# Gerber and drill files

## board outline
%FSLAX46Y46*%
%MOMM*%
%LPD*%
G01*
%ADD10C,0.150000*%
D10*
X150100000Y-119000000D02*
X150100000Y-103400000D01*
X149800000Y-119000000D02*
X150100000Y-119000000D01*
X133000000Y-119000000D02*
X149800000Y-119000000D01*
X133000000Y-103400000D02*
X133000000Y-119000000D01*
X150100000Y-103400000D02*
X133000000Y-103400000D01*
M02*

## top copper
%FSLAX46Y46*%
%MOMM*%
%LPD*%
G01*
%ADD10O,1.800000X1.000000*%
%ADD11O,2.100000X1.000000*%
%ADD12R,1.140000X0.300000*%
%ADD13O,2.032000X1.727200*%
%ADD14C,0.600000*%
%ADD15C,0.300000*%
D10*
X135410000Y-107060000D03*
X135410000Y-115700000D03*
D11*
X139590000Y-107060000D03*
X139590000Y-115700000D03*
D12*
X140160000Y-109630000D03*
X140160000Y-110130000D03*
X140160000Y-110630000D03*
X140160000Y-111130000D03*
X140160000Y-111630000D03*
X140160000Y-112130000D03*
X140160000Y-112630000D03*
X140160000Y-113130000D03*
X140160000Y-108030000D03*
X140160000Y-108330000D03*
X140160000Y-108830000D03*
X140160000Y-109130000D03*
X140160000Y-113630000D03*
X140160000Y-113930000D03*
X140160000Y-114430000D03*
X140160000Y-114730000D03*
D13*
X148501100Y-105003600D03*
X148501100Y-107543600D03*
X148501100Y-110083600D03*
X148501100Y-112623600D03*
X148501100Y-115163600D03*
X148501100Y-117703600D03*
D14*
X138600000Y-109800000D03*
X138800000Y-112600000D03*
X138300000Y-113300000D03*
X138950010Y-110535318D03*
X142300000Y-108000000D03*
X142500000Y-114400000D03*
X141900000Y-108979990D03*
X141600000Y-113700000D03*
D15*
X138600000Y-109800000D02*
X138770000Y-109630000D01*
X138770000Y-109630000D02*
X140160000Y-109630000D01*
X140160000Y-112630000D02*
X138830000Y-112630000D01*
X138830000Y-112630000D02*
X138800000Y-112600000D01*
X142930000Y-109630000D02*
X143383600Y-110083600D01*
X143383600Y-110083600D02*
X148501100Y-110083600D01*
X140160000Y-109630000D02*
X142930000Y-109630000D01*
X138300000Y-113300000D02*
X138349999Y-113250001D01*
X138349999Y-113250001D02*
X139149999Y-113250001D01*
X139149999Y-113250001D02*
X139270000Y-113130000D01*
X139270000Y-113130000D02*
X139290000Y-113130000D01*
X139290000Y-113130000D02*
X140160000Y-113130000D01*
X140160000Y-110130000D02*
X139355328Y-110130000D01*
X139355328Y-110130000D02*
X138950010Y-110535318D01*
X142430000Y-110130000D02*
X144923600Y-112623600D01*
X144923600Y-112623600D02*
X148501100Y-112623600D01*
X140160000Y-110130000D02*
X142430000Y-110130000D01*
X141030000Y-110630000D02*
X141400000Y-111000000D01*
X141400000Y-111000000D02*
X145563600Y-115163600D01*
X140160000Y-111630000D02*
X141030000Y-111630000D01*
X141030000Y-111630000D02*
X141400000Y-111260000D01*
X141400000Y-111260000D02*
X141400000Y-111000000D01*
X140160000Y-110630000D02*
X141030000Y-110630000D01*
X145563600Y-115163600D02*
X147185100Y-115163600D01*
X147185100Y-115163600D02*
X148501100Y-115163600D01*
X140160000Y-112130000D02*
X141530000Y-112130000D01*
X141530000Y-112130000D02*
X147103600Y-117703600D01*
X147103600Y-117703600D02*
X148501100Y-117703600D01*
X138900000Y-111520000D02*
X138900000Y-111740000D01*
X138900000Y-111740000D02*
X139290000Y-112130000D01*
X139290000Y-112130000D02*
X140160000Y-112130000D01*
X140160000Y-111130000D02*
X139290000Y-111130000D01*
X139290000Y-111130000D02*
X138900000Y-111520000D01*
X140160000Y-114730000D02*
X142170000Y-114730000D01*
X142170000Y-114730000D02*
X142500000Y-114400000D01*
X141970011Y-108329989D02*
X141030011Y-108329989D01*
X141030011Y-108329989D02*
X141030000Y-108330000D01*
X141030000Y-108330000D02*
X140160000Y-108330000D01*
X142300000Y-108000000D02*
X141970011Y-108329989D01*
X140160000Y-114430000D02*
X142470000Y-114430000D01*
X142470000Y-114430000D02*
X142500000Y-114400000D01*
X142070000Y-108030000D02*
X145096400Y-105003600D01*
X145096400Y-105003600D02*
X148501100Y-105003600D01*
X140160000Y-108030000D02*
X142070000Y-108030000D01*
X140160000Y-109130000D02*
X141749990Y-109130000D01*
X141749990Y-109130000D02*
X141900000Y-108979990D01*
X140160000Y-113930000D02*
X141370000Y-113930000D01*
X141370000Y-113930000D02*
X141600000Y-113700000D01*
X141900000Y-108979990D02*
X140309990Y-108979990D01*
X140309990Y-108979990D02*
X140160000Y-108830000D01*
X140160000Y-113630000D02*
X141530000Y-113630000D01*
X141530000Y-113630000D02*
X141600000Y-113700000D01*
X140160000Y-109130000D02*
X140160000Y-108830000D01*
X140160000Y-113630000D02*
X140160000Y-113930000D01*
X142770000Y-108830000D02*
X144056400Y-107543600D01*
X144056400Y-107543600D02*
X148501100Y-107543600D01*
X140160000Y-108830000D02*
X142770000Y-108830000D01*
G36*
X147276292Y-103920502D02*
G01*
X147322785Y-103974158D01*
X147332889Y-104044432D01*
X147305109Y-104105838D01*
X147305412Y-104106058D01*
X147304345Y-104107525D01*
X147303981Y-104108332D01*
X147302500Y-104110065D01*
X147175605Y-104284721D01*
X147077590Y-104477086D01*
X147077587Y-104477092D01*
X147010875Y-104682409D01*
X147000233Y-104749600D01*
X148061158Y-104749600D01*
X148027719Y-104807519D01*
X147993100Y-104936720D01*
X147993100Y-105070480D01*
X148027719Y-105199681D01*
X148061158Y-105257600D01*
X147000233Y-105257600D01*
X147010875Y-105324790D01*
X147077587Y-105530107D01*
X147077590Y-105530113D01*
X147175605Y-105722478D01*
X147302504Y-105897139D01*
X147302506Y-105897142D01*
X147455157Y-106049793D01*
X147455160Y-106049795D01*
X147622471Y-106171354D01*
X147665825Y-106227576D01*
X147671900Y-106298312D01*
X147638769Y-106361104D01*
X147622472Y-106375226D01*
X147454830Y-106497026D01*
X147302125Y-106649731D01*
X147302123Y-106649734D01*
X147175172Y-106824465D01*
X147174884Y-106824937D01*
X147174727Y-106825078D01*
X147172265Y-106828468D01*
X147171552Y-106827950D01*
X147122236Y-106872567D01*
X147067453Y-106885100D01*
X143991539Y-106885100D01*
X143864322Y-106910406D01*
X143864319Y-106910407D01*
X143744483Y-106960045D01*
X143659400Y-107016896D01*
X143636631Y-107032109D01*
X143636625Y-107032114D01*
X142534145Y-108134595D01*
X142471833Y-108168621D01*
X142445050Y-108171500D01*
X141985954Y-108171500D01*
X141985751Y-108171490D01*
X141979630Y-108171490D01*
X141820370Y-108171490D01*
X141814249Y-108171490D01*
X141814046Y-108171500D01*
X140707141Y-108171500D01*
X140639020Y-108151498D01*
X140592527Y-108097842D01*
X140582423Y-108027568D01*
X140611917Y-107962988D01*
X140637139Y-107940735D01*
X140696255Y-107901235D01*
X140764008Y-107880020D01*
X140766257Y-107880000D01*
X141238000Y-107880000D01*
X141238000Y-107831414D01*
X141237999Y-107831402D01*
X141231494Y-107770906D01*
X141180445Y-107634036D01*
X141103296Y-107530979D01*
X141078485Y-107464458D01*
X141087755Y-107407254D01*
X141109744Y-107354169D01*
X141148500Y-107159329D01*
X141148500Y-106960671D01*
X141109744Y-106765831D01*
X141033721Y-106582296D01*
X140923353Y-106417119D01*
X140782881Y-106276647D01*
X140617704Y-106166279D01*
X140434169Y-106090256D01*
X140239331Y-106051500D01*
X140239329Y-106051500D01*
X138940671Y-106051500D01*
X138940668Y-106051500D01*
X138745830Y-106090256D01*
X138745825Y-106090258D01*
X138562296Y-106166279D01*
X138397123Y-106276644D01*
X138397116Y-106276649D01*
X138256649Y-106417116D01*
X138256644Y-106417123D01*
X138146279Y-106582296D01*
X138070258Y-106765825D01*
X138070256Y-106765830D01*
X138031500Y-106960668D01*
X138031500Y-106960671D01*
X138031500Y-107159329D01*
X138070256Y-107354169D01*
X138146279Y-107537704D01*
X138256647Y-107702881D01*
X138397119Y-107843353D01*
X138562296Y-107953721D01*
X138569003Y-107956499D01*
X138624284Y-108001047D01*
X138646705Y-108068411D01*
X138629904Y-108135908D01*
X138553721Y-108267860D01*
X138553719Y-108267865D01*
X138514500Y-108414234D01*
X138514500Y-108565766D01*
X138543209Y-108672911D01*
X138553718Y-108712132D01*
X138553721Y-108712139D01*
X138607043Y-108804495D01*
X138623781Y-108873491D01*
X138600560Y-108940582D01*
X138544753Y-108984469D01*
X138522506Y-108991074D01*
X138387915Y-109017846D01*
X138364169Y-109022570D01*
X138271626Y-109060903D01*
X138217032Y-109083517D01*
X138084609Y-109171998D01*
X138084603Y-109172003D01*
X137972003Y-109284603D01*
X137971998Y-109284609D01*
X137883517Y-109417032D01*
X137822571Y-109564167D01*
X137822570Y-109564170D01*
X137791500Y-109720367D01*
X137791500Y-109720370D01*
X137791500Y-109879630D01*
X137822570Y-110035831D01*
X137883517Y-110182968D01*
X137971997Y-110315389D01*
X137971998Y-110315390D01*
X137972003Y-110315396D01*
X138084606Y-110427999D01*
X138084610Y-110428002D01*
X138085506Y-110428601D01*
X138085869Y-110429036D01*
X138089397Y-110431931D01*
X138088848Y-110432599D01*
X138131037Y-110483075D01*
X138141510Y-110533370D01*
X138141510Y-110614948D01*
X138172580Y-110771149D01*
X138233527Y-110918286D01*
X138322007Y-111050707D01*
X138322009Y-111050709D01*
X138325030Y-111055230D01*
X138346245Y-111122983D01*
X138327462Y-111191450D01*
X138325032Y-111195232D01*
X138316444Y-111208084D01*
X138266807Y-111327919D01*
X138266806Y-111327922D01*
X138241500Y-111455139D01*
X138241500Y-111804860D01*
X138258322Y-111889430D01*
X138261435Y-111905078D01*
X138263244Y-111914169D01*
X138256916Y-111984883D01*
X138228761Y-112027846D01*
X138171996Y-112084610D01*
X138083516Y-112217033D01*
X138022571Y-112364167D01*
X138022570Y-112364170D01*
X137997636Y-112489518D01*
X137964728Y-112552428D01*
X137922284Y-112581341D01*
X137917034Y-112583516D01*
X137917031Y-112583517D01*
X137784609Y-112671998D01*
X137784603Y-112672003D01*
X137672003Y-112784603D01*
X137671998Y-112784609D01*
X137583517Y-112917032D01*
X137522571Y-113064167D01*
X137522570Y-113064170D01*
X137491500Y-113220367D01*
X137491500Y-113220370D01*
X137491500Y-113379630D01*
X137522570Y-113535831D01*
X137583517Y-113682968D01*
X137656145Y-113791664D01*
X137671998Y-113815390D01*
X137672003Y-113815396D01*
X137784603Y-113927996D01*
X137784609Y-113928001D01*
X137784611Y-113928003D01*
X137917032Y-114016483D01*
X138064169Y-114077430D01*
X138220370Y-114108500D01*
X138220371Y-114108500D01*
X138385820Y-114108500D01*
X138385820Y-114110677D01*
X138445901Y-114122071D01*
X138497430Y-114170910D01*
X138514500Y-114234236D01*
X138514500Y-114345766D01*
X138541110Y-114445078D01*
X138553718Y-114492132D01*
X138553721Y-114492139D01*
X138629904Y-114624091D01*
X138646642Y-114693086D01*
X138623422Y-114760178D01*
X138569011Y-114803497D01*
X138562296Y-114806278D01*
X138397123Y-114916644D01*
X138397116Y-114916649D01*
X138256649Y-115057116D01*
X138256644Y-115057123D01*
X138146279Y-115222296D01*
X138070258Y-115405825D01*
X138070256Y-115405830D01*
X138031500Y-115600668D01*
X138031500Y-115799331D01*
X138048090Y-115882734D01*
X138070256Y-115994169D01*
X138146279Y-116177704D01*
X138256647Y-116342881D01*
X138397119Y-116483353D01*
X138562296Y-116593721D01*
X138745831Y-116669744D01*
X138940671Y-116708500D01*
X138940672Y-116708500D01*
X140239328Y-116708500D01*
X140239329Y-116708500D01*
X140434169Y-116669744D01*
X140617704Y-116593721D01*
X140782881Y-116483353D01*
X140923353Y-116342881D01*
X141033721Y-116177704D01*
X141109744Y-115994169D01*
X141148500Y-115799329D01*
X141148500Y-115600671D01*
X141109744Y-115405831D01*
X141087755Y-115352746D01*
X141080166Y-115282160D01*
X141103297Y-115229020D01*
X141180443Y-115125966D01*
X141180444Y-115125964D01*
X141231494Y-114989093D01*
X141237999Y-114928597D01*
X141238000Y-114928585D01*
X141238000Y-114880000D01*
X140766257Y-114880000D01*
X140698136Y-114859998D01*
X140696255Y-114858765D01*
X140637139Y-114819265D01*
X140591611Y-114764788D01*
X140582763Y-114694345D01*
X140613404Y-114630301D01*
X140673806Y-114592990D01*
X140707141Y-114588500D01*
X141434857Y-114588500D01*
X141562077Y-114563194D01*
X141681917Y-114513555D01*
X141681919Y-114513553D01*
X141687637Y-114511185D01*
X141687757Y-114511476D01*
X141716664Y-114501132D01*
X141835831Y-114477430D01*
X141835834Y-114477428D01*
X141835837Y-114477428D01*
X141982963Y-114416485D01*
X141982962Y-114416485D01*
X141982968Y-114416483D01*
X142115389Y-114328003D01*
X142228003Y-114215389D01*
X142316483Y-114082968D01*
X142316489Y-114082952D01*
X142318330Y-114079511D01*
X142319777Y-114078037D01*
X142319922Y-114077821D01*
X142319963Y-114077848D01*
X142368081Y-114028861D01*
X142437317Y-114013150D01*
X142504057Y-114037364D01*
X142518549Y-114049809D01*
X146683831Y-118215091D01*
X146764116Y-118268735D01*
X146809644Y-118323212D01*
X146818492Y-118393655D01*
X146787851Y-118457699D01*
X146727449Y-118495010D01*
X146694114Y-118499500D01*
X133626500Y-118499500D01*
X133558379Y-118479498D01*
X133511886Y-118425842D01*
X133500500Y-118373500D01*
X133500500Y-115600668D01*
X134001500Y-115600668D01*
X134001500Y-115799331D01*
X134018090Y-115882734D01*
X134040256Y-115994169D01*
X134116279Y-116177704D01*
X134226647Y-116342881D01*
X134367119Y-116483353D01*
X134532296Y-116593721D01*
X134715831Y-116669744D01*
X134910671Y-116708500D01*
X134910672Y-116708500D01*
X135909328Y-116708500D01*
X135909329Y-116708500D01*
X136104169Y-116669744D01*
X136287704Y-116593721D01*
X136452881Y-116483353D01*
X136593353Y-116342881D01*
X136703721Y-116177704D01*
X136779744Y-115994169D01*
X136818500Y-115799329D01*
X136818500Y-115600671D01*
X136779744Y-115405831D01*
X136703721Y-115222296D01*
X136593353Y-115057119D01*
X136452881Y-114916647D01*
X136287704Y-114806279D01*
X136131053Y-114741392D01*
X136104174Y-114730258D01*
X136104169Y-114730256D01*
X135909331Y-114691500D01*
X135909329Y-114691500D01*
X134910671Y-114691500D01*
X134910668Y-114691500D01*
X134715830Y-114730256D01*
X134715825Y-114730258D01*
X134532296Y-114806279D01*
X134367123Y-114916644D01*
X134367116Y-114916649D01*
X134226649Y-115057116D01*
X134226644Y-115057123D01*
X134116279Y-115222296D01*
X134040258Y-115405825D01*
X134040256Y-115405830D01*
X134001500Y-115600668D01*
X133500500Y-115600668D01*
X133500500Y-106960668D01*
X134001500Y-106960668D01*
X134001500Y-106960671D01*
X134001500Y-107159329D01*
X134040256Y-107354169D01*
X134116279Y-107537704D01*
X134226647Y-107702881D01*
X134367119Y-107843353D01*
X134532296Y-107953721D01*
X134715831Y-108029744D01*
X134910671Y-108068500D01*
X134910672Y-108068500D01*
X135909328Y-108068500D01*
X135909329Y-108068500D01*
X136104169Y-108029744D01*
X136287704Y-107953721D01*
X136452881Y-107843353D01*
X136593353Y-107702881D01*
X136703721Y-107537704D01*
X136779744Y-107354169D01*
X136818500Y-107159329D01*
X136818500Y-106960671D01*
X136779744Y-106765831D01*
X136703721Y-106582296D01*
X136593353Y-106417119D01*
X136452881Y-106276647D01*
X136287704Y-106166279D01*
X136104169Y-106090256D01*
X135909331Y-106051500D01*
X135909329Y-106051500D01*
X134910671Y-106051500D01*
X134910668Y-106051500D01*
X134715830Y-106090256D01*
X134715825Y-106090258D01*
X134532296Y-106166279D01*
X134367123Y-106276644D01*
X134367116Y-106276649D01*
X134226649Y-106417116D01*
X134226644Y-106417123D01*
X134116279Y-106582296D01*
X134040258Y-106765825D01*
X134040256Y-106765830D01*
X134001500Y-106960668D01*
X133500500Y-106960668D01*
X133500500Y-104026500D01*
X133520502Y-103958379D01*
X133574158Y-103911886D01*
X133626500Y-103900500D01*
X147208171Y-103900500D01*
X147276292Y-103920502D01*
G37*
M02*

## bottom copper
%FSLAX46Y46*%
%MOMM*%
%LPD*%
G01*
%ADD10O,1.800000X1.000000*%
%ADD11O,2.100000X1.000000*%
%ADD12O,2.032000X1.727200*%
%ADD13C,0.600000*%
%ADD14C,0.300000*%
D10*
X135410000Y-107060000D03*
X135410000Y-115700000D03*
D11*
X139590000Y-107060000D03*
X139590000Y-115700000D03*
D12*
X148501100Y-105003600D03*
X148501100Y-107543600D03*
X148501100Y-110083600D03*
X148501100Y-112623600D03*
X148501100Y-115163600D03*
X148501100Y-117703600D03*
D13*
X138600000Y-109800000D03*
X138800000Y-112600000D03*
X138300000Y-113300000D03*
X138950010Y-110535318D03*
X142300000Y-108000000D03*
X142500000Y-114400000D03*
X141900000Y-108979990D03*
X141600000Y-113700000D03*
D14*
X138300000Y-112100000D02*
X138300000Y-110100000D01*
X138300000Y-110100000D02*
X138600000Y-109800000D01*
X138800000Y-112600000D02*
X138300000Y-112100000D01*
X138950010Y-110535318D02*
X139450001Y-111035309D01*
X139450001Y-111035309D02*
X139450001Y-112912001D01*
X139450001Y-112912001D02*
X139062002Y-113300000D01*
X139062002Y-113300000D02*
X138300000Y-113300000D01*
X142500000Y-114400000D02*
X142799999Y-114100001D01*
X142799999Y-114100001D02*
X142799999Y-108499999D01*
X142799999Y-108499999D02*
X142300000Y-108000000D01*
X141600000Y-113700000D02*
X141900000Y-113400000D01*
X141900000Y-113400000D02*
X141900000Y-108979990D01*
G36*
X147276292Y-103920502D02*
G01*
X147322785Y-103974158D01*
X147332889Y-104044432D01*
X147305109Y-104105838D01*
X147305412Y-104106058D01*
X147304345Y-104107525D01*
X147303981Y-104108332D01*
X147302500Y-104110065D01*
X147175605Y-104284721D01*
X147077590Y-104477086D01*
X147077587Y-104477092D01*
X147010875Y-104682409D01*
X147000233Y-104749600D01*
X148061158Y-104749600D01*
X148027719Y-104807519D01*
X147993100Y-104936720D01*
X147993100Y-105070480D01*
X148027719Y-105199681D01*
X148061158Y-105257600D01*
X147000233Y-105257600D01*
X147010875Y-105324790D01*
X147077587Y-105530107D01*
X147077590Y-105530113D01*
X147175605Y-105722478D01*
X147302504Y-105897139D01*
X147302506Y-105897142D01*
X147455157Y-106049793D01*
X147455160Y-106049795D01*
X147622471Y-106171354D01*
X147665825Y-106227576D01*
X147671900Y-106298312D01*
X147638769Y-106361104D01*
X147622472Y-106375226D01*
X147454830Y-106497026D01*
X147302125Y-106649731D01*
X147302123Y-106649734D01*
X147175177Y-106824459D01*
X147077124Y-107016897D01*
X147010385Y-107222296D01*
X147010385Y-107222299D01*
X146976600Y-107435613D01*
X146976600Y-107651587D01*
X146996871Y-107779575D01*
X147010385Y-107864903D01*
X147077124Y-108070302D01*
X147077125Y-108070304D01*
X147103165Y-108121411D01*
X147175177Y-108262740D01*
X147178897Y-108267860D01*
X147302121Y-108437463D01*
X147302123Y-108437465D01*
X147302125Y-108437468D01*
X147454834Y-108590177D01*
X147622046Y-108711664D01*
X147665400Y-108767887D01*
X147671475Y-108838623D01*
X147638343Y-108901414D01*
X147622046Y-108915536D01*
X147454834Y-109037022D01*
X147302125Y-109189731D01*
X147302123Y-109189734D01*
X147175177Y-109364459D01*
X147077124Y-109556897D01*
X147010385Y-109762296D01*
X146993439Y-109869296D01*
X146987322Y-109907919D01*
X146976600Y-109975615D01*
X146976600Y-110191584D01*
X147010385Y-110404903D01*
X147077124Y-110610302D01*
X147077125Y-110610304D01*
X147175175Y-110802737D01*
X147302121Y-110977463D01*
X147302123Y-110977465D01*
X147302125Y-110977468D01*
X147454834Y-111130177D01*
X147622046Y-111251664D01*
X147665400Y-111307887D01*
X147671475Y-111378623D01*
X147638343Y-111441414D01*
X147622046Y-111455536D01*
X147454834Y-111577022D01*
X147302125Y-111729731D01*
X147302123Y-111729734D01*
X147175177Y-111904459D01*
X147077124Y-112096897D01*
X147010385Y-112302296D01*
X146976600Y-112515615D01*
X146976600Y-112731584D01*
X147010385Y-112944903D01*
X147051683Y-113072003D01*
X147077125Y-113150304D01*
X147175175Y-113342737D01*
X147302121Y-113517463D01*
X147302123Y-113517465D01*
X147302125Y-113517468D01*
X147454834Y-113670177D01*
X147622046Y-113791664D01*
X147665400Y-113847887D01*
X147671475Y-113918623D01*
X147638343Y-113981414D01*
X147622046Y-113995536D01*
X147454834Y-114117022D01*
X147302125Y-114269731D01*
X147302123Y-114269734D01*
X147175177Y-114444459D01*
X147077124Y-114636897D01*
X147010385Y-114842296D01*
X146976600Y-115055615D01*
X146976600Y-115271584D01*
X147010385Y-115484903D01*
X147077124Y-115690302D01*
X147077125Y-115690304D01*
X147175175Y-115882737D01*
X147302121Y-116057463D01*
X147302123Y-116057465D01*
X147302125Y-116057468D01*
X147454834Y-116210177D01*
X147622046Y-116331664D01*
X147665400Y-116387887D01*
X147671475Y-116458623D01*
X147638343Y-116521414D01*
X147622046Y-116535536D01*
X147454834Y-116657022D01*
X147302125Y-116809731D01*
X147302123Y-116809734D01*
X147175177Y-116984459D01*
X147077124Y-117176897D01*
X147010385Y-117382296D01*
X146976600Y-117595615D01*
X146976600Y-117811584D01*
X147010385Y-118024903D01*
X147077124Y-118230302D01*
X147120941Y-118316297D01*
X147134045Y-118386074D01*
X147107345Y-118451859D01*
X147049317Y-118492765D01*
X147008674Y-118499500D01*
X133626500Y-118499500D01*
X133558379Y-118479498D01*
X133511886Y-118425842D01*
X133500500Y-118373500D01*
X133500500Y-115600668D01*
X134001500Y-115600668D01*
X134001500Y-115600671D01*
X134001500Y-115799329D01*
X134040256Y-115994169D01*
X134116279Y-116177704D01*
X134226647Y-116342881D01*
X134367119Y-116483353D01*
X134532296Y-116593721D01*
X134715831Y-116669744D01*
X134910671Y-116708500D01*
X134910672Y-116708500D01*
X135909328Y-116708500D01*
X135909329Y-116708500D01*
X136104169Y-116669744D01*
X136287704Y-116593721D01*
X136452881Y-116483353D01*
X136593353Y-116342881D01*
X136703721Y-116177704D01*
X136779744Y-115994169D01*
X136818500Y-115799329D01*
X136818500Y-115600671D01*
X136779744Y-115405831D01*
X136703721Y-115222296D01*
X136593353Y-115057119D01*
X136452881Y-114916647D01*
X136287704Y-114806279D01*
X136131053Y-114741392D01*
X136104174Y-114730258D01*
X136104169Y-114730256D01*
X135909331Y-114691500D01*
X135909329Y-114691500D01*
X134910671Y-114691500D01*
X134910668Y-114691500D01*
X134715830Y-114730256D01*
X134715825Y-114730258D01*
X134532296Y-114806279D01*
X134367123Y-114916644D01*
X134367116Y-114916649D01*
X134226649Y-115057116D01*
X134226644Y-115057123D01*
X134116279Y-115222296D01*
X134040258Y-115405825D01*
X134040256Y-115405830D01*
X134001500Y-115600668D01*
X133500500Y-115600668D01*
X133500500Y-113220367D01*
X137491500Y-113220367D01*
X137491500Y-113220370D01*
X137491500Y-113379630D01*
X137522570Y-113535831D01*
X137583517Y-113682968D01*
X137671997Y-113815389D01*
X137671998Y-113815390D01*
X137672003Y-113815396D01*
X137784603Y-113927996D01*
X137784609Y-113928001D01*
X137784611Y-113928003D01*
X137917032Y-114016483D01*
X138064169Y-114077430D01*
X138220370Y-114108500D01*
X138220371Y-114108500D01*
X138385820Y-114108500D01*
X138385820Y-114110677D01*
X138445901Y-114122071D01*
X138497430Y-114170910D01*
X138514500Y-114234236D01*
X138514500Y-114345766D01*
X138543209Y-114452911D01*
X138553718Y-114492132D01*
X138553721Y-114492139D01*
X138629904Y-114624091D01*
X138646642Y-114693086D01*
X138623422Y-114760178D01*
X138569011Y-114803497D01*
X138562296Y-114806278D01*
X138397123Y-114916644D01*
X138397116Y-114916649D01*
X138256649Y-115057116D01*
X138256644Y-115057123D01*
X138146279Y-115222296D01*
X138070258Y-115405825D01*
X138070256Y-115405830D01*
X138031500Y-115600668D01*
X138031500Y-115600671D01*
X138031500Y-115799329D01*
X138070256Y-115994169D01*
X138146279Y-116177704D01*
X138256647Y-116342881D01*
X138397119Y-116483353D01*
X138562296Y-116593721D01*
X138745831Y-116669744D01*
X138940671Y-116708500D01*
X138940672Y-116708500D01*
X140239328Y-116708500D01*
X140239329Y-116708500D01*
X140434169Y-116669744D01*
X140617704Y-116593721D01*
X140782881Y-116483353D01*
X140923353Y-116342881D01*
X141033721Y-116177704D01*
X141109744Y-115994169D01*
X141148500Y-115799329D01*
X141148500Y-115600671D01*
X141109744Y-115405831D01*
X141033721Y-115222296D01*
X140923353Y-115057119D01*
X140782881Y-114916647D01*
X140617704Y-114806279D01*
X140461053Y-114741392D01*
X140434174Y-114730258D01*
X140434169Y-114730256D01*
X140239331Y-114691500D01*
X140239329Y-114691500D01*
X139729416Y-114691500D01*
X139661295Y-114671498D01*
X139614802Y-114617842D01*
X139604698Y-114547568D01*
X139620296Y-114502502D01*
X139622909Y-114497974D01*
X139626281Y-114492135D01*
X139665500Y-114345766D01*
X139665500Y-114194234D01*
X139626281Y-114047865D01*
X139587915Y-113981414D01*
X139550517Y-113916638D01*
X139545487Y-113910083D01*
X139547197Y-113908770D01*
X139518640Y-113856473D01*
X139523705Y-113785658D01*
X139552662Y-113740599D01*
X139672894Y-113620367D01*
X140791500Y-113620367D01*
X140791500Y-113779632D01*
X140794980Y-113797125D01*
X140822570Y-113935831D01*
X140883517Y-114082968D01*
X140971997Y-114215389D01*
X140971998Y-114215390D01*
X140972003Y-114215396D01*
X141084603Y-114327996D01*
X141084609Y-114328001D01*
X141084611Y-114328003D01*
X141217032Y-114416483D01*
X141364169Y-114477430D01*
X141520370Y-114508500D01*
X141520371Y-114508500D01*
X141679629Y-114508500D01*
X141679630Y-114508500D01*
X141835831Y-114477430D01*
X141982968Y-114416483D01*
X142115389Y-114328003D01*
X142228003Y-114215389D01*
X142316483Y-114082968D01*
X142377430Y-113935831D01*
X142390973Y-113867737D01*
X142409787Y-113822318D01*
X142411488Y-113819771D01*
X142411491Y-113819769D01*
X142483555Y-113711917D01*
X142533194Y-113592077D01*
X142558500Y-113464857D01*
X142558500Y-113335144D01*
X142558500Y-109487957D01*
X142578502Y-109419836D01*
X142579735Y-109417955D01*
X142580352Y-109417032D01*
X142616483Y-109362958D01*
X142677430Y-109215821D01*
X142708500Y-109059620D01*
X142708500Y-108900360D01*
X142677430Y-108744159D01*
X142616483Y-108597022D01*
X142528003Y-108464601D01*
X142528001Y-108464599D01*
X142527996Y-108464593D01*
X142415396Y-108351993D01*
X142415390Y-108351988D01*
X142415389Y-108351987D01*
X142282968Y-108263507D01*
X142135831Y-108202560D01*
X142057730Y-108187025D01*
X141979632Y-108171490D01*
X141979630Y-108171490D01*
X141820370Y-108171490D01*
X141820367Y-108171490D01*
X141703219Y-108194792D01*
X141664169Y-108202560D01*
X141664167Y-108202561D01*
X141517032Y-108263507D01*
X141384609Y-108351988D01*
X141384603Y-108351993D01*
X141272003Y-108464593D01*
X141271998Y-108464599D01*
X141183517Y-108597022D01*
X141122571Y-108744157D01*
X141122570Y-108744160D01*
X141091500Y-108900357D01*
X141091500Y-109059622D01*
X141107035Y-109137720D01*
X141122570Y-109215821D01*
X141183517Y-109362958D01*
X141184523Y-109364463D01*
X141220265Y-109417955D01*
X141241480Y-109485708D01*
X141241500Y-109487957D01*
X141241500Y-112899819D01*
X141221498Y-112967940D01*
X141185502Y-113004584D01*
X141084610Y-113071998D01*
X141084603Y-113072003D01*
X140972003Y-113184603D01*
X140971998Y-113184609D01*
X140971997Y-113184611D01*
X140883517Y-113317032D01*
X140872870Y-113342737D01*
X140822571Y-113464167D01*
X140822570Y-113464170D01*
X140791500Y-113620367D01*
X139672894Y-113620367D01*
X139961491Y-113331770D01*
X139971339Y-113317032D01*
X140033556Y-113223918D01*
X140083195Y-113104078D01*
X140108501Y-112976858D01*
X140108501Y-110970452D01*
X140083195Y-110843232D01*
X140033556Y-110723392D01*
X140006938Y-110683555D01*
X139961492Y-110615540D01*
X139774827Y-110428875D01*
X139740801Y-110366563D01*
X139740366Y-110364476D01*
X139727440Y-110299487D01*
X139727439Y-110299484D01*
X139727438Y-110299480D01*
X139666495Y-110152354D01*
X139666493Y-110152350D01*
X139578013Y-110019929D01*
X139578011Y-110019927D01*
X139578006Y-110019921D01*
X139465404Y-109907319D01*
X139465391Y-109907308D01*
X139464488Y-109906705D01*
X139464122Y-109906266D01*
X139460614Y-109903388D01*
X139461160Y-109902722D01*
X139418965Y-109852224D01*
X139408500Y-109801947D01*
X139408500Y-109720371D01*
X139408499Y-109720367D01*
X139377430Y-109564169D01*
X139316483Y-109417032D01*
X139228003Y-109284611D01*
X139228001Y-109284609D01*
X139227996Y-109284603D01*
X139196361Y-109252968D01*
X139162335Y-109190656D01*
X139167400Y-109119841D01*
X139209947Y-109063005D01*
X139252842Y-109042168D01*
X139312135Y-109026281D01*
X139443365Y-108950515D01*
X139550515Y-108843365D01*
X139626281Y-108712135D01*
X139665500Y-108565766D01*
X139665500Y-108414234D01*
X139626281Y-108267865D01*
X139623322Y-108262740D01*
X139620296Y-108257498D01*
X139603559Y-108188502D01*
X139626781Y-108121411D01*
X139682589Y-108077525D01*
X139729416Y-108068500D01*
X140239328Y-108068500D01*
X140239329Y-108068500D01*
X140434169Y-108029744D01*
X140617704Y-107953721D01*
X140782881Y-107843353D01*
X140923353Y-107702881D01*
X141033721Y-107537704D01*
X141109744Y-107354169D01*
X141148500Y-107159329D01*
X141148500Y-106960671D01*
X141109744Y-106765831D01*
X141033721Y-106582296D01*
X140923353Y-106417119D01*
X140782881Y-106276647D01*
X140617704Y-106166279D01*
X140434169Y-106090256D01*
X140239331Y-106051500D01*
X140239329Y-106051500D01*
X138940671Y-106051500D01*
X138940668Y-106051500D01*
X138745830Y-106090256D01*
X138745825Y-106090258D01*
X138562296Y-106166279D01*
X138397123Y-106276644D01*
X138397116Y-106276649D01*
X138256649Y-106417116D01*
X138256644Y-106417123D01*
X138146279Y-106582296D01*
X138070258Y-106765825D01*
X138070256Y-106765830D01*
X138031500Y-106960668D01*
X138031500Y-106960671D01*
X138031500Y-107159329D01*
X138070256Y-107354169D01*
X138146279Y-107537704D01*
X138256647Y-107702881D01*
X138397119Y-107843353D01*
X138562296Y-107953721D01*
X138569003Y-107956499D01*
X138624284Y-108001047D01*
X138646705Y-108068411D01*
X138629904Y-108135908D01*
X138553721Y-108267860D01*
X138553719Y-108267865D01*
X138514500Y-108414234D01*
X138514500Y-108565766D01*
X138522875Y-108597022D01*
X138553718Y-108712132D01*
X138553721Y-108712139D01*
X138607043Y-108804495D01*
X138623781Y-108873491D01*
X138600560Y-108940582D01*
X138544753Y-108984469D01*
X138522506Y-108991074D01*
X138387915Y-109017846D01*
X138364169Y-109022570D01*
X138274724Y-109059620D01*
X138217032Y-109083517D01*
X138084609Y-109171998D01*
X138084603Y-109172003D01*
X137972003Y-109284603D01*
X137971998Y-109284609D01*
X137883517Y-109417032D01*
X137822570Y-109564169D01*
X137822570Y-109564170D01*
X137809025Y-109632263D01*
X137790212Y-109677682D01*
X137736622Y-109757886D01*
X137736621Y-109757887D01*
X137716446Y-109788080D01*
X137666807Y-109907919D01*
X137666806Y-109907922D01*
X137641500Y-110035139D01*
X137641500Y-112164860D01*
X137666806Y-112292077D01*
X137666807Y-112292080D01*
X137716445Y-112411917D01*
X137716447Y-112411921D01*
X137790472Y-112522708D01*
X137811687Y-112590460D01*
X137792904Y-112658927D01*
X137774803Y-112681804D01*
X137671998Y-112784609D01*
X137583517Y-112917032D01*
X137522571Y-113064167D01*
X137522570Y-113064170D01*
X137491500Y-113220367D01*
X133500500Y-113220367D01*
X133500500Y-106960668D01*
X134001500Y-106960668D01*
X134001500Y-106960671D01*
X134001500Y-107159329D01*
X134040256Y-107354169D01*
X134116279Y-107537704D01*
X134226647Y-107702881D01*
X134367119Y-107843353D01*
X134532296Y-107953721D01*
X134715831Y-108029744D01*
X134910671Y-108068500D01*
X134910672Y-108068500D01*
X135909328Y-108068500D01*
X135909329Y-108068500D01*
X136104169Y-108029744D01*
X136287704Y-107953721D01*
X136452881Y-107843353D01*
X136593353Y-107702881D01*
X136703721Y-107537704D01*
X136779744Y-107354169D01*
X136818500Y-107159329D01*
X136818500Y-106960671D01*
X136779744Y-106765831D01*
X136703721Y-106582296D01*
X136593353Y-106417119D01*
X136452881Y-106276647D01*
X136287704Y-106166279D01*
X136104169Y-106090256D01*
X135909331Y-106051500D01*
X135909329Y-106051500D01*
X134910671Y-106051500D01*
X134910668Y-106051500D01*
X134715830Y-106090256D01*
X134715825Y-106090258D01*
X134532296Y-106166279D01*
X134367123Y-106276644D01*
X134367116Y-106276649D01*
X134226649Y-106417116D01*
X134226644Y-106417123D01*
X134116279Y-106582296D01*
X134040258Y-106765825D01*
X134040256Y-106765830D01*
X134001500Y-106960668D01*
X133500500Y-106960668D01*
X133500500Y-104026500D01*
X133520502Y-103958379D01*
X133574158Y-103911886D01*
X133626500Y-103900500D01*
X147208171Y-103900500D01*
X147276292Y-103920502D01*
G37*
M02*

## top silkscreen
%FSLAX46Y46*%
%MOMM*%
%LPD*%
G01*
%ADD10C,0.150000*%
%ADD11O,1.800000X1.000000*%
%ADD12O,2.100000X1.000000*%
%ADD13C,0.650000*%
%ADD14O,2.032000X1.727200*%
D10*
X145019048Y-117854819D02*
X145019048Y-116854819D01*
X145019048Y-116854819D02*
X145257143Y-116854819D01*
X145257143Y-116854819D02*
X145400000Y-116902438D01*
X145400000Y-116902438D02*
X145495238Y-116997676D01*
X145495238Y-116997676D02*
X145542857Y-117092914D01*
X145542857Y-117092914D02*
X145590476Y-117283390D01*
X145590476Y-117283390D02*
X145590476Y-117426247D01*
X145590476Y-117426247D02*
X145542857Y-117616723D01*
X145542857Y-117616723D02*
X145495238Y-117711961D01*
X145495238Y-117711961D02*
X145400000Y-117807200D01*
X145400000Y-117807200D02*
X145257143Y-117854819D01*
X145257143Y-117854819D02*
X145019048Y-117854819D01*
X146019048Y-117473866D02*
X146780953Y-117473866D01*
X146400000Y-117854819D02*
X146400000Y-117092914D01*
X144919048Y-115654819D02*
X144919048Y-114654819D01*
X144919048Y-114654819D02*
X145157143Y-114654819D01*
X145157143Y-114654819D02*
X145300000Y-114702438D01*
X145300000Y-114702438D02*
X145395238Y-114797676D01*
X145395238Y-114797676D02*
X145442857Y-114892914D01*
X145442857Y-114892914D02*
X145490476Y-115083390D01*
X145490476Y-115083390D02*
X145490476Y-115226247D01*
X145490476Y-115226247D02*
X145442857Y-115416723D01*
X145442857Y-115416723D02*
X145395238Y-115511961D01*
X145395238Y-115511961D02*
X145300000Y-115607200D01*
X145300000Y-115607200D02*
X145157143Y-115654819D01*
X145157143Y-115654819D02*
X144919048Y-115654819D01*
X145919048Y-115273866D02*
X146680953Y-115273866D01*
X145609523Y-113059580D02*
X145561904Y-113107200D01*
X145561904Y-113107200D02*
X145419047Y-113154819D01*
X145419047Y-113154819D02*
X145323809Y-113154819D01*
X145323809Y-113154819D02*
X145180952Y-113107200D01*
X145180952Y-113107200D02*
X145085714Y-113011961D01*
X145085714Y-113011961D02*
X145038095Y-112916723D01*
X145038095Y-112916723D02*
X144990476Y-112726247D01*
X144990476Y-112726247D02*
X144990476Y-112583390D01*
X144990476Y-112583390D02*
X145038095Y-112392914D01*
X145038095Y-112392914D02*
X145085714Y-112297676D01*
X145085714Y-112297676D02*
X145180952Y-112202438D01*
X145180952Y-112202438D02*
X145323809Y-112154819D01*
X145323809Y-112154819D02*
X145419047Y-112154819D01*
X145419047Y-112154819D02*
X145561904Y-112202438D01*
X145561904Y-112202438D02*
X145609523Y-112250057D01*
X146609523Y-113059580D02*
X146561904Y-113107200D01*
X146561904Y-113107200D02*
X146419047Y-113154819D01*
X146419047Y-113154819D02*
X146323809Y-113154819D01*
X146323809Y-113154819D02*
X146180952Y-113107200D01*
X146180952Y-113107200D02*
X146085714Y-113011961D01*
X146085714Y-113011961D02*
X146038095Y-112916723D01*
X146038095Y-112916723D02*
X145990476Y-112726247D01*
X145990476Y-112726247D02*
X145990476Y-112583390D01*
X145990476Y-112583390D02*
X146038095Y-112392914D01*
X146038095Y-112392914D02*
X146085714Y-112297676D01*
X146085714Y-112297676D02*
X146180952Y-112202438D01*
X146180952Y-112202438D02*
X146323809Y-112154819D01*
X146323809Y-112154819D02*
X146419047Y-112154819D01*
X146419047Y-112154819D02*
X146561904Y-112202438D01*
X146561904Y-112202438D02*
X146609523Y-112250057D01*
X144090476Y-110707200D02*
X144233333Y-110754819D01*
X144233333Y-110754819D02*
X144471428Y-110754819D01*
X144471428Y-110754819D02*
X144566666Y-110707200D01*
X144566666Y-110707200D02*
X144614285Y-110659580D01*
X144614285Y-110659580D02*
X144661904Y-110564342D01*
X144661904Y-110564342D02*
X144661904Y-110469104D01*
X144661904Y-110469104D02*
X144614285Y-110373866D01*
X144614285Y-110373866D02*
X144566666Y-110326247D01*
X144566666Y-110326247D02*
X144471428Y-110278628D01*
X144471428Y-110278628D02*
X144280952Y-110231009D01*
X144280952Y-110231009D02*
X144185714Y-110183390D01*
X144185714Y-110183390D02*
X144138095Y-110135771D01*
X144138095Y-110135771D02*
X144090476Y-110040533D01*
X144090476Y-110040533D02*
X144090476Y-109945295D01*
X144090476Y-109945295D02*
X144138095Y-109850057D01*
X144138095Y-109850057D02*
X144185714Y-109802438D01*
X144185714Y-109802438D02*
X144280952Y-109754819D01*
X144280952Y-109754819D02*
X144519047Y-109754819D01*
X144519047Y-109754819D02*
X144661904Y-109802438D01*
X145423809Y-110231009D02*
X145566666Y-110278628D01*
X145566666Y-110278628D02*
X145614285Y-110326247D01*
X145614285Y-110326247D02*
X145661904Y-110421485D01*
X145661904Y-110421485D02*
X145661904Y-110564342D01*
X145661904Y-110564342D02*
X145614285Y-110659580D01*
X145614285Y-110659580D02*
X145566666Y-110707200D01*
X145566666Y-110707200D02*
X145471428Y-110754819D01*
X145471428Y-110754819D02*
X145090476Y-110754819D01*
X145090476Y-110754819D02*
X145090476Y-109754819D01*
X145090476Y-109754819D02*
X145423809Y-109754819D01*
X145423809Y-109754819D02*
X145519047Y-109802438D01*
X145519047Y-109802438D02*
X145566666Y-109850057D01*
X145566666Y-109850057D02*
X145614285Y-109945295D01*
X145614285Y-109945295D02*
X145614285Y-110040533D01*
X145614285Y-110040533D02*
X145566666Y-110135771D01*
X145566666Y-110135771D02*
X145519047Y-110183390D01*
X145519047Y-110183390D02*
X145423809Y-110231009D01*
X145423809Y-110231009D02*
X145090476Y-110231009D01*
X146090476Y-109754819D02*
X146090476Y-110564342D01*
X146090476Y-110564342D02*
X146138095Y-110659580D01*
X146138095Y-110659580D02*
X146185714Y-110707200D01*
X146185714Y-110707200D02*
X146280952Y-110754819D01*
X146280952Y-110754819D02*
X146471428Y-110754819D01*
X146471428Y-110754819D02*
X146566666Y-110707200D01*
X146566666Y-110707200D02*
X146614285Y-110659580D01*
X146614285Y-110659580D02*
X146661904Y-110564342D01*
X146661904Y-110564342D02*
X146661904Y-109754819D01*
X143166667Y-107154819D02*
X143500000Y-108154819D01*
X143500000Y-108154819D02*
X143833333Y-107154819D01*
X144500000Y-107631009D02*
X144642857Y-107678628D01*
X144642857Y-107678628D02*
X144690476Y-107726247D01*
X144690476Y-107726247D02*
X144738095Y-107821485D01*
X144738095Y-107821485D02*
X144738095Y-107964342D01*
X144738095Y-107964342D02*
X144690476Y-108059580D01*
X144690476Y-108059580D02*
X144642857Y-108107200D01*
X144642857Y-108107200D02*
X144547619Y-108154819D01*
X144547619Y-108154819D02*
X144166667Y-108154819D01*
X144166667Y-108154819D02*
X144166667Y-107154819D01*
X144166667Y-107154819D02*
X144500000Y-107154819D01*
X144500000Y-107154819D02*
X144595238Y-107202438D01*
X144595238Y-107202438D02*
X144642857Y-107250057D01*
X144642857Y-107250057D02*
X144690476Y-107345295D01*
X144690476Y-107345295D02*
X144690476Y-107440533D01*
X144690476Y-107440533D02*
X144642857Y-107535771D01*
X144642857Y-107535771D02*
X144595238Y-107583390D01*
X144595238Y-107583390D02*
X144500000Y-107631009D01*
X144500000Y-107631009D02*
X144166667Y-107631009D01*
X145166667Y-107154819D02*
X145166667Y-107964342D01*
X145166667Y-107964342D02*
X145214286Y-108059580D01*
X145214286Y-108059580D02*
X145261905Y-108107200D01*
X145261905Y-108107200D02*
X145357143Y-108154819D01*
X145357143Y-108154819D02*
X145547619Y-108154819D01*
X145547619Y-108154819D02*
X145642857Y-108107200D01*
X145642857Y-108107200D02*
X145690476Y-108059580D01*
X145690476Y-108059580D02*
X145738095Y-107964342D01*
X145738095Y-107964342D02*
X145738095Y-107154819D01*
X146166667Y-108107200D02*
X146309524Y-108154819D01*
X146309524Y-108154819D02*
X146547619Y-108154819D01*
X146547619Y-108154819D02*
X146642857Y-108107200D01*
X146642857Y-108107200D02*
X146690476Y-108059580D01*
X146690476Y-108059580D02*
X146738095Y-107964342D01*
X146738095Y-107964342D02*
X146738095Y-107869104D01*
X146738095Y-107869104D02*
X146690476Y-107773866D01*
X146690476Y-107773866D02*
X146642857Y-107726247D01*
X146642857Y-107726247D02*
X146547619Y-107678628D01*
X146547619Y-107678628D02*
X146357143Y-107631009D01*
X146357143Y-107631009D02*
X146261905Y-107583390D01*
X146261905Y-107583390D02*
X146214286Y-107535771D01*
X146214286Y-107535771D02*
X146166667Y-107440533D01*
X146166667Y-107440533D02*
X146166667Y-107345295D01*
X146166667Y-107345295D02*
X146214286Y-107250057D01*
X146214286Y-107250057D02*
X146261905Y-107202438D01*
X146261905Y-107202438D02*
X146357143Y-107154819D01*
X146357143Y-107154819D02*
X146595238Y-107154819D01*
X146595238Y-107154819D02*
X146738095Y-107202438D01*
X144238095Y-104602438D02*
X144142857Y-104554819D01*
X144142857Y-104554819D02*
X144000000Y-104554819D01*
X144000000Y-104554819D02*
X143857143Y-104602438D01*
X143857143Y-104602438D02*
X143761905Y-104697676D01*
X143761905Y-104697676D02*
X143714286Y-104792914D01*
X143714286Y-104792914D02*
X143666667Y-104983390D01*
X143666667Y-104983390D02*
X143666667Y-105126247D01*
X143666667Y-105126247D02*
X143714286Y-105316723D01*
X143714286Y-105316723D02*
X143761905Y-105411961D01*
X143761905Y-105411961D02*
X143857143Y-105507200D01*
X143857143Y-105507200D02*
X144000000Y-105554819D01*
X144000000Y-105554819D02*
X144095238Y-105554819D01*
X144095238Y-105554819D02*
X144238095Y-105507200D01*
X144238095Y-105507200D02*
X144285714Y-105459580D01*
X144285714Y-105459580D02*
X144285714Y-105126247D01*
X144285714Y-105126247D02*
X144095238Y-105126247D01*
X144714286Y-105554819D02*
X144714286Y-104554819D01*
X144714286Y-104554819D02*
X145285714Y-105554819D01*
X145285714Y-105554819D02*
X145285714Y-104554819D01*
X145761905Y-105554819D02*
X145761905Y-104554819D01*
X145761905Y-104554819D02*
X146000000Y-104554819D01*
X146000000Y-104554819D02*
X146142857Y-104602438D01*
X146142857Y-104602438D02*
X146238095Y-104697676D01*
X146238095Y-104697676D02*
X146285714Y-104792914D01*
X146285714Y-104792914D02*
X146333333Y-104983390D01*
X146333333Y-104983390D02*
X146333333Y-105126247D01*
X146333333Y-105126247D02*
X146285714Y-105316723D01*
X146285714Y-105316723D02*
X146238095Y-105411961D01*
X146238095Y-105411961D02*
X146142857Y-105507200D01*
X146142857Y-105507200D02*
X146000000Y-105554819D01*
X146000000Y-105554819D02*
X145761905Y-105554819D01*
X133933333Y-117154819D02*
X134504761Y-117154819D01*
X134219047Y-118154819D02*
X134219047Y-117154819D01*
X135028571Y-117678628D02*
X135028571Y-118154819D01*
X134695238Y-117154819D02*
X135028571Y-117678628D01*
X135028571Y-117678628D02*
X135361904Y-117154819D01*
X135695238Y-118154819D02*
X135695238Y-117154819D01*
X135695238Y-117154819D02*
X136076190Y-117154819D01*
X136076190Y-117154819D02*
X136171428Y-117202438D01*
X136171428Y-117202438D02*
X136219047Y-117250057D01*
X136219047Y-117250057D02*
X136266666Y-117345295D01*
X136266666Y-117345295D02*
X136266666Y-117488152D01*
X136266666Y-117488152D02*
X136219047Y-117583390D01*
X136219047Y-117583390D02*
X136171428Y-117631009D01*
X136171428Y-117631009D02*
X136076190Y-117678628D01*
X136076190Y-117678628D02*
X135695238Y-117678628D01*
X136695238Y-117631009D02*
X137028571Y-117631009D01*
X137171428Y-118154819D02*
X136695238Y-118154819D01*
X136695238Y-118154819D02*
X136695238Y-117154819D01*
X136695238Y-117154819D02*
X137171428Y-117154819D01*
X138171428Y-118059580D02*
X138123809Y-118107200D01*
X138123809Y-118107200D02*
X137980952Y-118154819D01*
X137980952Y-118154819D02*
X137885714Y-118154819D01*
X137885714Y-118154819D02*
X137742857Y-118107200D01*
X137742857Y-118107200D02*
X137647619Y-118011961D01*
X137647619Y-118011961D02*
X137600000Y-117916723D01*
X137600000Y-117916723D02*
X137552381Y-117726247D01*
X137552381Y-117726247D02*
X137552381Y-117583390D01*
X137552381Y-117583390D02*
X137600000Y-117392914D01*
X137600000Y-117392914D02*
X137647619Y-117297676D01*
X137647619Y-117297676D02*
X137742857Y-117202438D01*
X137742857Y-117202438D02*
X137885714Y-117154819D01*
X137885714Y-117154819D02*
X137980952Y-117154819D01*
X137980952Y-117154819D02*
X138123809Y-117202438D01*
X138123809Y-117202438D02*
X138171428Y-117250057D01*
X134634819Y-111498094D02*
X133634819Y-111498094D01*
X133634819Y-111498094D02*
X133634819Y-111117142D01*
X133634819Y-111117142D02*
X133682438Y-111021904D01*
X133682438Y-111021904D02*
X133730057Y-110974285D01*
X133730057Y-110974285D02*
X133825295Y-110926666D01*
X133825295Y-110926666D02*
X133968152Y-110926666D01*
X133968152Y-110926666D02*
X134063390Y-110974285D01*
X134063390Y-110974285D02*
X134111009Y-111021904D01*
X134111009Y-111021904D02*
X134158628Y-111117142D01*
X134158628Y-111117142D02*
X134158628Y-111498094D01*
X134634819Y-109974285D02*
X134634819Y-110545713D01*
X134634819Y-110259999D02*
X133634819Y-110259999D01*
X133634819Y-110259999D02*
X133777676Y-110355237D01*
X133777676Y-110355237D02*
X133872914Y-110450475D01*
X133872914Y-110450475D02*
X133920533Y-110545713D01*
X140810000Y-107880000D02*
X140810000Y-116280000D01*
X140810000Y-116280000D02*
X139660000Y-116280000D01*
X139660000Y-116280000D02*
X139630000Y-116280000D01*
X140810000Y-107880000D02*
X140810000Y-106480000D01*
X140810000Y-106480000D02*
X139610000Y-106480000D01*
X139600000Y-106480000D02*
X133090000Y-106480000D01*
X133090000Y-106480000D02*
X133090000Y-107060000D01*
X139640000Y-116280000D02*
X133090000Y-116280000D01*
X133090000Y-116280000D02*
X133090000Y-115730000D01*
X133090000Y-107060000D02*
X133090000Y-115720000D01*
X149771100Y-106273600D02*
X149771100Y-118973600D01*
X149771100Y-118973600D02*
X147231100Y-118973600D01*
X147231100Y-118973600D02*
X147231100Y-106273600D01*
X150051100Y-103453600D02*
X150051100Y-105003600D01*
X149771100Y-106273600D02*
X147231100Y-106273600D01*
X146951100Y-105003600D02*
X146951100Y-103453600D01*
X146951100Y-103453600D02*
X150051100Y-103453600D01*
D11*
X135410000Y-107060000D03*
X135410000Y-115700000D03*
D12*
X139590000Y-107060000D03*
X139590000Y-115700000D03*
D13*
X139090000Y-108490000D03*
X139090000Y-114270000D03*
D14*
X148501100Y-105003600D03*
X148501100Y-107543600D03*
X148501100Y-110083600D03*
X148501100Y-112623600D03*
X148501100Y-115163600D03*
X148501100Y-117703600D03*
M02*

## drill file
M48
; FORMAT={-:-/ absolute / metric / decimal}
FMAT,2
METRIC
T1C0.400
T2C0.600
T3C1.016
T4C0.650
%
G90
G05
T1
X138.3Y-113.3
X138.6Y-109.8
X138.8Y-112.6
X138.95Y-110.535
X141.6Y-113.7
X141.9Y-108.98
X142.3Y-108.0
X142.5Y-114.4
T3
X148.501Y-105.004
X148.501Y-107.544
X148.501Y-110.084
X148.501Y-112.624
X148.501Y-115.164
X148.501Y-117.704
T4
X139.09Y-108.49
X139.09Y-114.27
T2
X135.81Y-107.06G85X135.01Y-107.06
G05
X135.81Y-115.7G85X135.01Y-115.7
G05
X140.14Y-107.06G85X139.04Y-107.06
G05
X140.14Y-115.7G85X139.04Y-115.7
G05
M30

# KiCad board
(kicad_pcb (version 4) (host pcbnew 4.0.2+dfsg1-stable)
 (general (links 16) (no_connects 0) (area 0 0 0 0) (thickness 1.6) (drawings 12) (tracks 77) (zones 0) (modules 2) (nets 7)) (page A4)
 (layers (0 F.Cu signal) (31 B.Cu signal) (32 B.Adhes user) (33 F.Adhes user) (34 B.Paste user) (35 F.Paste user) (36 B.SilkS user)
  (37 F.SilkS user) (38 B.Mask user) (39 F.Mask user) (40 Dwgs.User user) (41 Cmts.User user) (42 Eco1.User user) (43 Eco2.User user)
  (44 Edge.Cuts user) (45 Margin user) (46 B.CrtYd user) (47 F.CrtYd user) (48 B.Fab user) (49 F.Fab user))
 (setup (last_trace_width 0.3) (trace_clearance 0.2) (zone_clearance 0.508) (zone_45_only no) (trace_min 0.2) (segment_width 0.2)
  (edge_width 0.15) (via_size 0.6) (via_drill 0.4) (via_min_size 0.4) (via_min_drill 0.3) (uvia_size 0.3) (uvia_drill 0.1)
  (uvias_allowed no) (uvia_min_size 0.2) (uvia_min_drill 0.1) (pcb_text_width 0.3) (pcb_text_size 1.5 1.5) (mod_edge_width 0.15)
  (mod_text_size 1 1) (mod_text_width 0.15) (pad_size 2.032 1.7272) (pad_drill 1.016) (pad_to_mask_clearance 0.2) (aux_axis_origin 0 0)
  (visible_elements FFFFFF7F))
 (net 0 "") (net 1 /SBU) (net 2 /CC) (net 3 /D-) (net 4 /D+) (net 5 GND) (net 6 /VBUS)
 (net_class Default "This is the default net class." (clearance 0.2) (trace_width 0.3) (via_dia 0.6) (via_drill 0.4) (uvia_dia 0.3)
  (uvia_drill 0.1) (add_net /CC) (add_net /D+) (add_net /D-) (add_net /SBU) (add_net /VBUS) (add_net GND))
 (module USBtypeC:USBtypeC (layer F.Cu) (at 136.8 111.7 270)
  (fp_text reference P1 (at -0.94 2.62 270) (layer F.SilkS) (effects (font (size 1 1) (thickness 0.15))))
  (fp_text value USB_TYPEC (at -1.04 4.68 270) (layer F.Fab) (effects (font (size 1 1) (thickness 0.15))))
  (fp_line (start -3.82 -4.01) (end 4.58 -4.01) (layer F.SilkS) (width 0.15))
  (fp_line (start 4.58 -4.01) (end 4.58 -2.86) (layer F.SilkS) (width 0.15))
  (fp_line (start 4.58 -2.86) (end 4.58 -2.83) (layer F.SilkS) (width 0.15))
  (fp_line (start -3.82 -4.01) (end -5.22 -4.01) (layer F.SilkS) (width 0.15))
  (fp_line (start -5.22 -4.01) (end -5.22 -2.81) (layer F.SilkS) (width 0.15))
  (fp_line (start -5.22 -2.8) (end -5.22 3.71) (layer F.SilkS) (width 0.15))
  (fp_line (start -5.22 3.71) (end -4.64 3.71) (layer F.SilkS) (width 0.15))
  (fp_line (start 4.58 -2.84) (end 4.58 3.71) (layer F.SilkS) (width 0.15))
  (fp_line (start 4.58 3.71) (end 4.03 3.71) (layer F.SilkS) (width 0.15))
  (fp_line (start -4.64 3.71) (end 4.02 3.71) (layer F.SilkS) (width 0.15))
  (pad 1 thru_hole oval (at -4.64 1.39 270) (size 1 1.8) (drill oval 0.6 1.4) (layers *.Cu *.Mask F.SilkS))
  (pad 2 thru_hole oval (at 4 1.39 270) (size 1 1.8) (drill oval 0.6 1.4) (layers *.Cu *.Mask F.SilkS))
  (pad 3 thru_hole oval (at -4.64 -2.79 270) (size 1 2.1) (drill oval 0.6 1.7) (layers *.Cu *.Mask F.SilkS))
  (pad 4 thru_hole oval (at 4 -2.79 270) (size 1 2.1) (drill oval 0.6 1.7) (layers *.Cu *.Mask F.SilkS))
  (pad "" np_thru_hole circle (at -3.21 -2.29 270) (size 0.65 0.65) (drill 0.65) (layers *.Cu *.Mask F.SilkS))
  (pad "" np_thru_hole circle (at 2.57 -2.29 270) (size 0.65 0.65) (drill 0.65) (layers *.Cu *.Mask F.SilkS))
  (pad B8 smd rect (at -2.07 -3.36 270) (size 0.3 1.14) (layers F.Cu F.Paste F.Mask) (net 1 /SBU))
  (pad A5 smd rect (at -1.57 -3.36 270) (size 0.3 1.14) (layers F.Cu F.Paste F.Mask) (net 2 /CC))
  (pad B7 smd rect (at -1.07 -3.36 270) (size 0.3 1.14) (layers F.Cu F.Paste F.Mask) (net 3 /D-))
  (pad A6 smd rect (at -0.57 -3.36 270) (size 0.3 1.14) (layers F.Cu F.Paste F.Mask) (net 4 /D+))
  (pad A7 smd rect (at -0.07 -3.36 270) (size 0.3 1.14) (layers F.Cu F.Paste F.Mask) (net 3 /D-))
  (pad B6 smd rect (at 0.43 -3.36 270) (size 0.3 1.14) (layers F.Cu F.Paste F.Mask) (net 4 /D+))
  (pad A8 smd rect (at 0.93 -3.36 270) (size 0.3 1.14) (layers F.Cu F.Paste F.Mask) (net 1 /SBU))
  (pad B5 smd rect (at 1.43 -3.36 270) (size 0.3 1.14) (layers F.Cu F.Paste F.Mask) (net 2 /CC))
  (pad A1 smd rect (at -3.67 -3.36 270) (size 0.3 1.14) (layers F.Cu F.Paste F.Mask) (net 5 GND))
  (pad B12 smd rect (at -3.37 -3.36 270) (size 0.3 1.14) (layers F.Cu F.Paste F.Mask) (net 5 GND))
  (pad A4 smd rect (at -2.87 -3.36 270) (size 0.3 1.14) (layers F.Cu F.Paste F.Mask) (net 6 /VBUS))
  (pad B9 smd rect (at -2.57 -3.36 270) (size 0.3 1.14) (layers F.Cu F.Paste F.Mask) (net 6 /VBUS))
  (pad B4 smd rect (at 1.93 -3.36 270) (size 0.3 1.14) (layers F.Cu F.Paste F.Mask) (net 6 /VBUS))
  (pad A9 smd rect (at 2.23 -3.36 270) (size 0.3 1.14) (layers F.Cu F.Paste F.Mask) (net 6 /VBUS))
  (pad B1 smd rect (at 2.73 -3.36 270) (size 0.3 1.14) (layers F.Cu F.Paste F.Mask) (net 5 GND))
  (pad A12 smd rect (at 3.03 -3.36 270) (size 0.3 1.14) (layers F.Cu F.Paste F.Mask) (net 5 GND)))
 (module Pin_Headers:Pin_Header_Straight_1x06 (layer F.Cu) (at 148.5011 105.0036)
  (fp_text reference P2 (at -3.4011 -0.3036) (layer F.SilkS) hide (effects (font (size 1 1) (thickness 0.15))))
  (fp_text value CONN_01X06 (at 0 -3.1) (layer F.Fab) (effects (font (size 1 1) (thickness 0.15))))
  (fp_line (start 1.27 1.27) (end 1.27 13.97) (layer F.SilkS) (width 0.15))
  (fp_line (start 1.27 13.97) (end -1.27 13.97) (layer F.SilkS) (width 0.15))
  (fp_line (start -1.27 13.97) (end -1.27 1.27) (layer F.SilkS) (width 0.15))
  (fp_line (start 1.55 -1.55) (end 1.55 0) (layer F.SilkS) (width 0.15))
  (fp_line (start 1.27 1.27) (end -1.27 1.27) (layer F.SilkS) (width 0.15))
  (fp_line (start -1.55 0) (end -1.55 -1.55) (layer F.SilkS) (width 0.15))
  (fp_line (start -1.55 -1.55) (end 1.55 -1.55) (layer F.SilkS) (width 0.15))
  (pad 1 thru_hole oval (at 0 0) (size 2.032 1.7272) (drill 1.016) (layers *.Cu *.Mask F.SilkS) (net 5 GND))
  (pad 2 thru_hole oval (at 0 2.54) (size 2.032 1.7272) (drill 1.016) (layers *.Cu *.Mask F.SilkS) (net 6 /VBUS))
  (pad 3 thru_hole oval (at 0 5.08) (size 2.032 1.7272) (drill 1.016) (layers *.Cu *.Mask F.SilkS) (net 1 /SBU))
  (pad 4 thru_hole oval (at 0 7.62) (size 2.032 1.7272) (drill 1.016) (layers *.Cu *.Mask F.SilkS) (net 2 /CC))
  (pad 5 thru_hole oval (at 0 10.16) (size 2.032 1.7272) (drill 1.016) (layers *.Cu *.Mask F.SilkS) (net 3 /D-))
  (pad 6 thru_hole oval (at 0 12.7) (size 2.032 1.7272) (drill 1.016) (layers *.Cu *.Mask F.SilkS) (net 4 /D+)))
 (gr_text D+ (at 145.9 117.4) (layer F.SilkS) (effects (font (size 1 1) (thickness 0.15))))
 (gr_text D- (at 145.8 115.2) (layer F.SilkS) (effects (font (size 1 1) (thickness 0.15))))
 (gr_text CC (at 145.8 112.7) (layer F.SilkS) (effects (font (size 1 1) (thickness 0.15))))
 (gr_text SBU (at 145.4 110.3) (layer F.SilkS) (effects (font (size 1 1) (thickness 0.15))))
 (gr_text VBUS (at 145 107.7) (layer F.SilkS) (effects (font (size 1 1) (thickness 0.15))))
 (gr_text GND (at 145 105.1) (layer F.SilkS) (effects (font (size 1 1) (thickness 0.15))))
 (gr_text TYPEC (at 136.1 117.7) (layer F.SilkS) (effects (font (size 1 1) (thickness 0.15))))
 (gr_line (start 150.1 119) (end 150.1 103.4) (angle 90) (layer Edge.Cuts) (width 0.15))
 (gr_line (start 149.8 119) (end 150.1 119) (angle 90) (layer Edge.Cuts) (width 0.15))
 (gr_line (start 133 119) (end 149.8 119) (angle 90) (layer Edge.Cuts) (width 0.15))
 (gr_line (start 133 103.4) (end 133 119) (angle 90) (layer Edge.Cuts) (width 0.15))
 (gr_line (start 150.1 103.4) (end 133 103.4) (angle 90) (layer Edge.Cuts) (width 0.15))
 (segment (start 138.6 109.8) (end 138.77 109.63) (width 0.3) (layer F.Cu) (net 1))
 (segment (start 138.77 109.63) (end 140.16 109.63) (width 0.3) (layer F.Cu) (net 1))
 (segment (start 138.3 112.1) (end 138.3 110.1) (width 0.3) (layer B.Cu) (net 1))
 (segment (start 138.3 110.1) (end 138.6 109.8) (width 0.3) (layer B.Cu) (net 1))
 (via (at 138.6 109.8) (size 0.6) (drill 0.4) (layers F.Cu B.Cu) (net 1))
 (segment (start 138.8 112.6) (end 138.3 112.1) (width 0.3) (layer B.Cu) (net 1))
 (segment (start 140.16 112.63) (end 138.83 112.63) (width 0.3) (layer F.Cu) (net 1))
 (segment (start 138.83 112.63) (end 138.8 112.6) (width 0.3) (layer F.Cu) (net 1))
 (via (at 138.8 112.6) (size 0.6) (drill 0.4) (layers F.Cu B.Cu) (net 1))
 (segment (start 142.93 109.63) (end 143.3836 110.0836) (width 0.3) (layer F.Cu) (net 1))
 (segment (start 143.3836 110.0836) (end 148.5011 110.0836) (width 0.3) (layer F.Cu) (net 1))
 (segment (start 140.16 109.63) (end 142.93 109.63) (width 0.3) (layer F.Cu) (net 1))
 (segment (start 138.3 113.3) (end 138.349999 113.250001) (width 0.3) (layer F.Cu) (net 2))
 (segment (start 138.349999 113.250001) (end 139.149999 113.250001) (width 0.3) (layer F.Cu) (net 2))
 (segment (start 139.149999 113.250001) (end 139.27 113.13) (width 0.3) (layer F.Cu) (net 2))
 (segment (start 139.27 113.13) (end 139.29 113.13) (width 0.3) (layer F.Cu) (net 2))
 (segment (start 139.29 113.13) (end 140.16 113.13) (width 0.3) (layer F.Cu) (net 2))
 (segment (start 138.95001 110.535318) (end 139.450001 111.035309) (width 0.3) (layer B.Cu) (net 2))
 (segment (start 139.450001 111.035309) (end 139.450001 112.912001) (width 0.3) (layer B.Cu) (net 2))
 (segment (start 139.450001 112.912001) (end 139.062002 113.3) (width 0.3) (layer B.Cu) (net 2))
 (segment (start 139.062002 113.3) (end 138.3 113.3) (width 0.3) (layer B.Cu) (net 2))
 (via (at 138.3 113.3) (size 0.6) (drill 0.4) (layers F.Cu B.Cu) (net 2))
 (segment (start 140.16 110.13) (end 139.355328 110.13) (width 0.3) (layer F.Cu) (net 2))
 (segment (start 139.355328 110.13) (end 138.95001 110.535318) (width 0.3) (layer F.Cu) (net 2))
 (via (at 138.95001 110.535318) (size 0.6) (drill 0.4) (layers F.Cu B.Cu) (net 2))
 (segment (start 142.43 110.13) (end 144.9236 112.6236) (width 0.3) (layer F.Cu) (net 2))
 (segment (start 144.9236 112.6236) (end 148.5011 112.6236) (width 0.3) (layer F.Cu) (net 2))
 (segment (start 140.16 110.13) (end 142.43 110.13) (width 0.3) (layer F.Cu) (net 2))
 (segment (start 141.03 110.63) (end 141.4 111) (width 0.3) (layer F.Cu) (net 3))
 (segment (start 141.4 111) (end 145.5636 115.1636) (width 0.3) (layer F.Cu) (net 3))
 (segment (start 140.16 111.63) (end 141.03 111.63) (width 0.3) (layer F.Cu) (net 3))
 (segment (start 141.03 111.63) (end 141.4 111.26) (width 0.3) (layer F.Cu) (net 3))
 (segment (start 141.4 111.26) (end 141.4 111) (width 0.3) (layer F.Cu) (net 3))
 (segment (start 140.16 110.63) (end 141.03 110.63) (width 0.3) (layer F.Cu) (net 3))
 (segment (start 145.5636 115.1636) (end 147.1851 115.1636) (width 0.3) (layer F.Cu) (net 3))
 (segment (start 147.1851 115.1636) (end 148.5011 115.1636) (width 0.3) (layer F.Cu) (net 3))
 (segment (start 140.16 112.13) (end 141.53 112.13) (width 0.3) (layer F.Cu) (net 4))
 (segment (start 141.53 112.13) (end 147.1036 117.7036) (width 0.3) (layer F.Cu) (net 4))
 (segment (start 147.1036 117.7036) (end 148.5011 117.7036) (width 0.3) (layer F.Cu) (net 4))
 (segment (start 138.9 111.52) (end 138.9 111.74) (width 0.3) (layer F.Cu) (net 4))
 (segment (start 138.9 111.74) (end 139.29 112.13) (width 0.3) (layer F.Cu) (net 4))
 (segment (start 139.29 112.13) (end 140.16 112.13) (width 0.3) (layer F.Cu) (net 4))
 (segment (start 140.16 111.13) (end 139.29 111.13) (width 0.3) (layer F.Cu) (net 4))
 (segment (start 139.29 111.13) (end 138.9 111.52) (width 0.3) (layer F.Cu) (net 4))
 (segment (start 140.16 114.73) (end 142.17 114.73) (width 0.3) (layer F.Cu) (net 5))
 (segment (start 142.17 114.73) (end 142.5 114.4) (width 0.3) (layer F.Cu) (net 5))
 (segment (start 141.970011 108.329989) (end 141.030011 108.329989) (width 0.3) (layer F.Cu) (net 5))
 (segment (start 141.030011 108.329989) (end 141.03 108.33) (width 0.3) (layer F.Cu) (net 5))
 (segment (start 141.03 108.33) (end 140.16 108.33) (width 0.3) (layer F.Cu) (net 5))
 (segment (start 142.3 108) (end 141.970011 108.329989) (width 0.3) (layer F.Cu) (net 5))
 (segment (start 142.5 114.4) (end 142.799999 114.100001) (width 0.3) (layer B.Cu) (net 5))
 (segment (start 142.799999 114.100001) (end 142.799999 108.499999) (width 0.3) (layer B.Cu) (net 5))
 (segment (start 142.799999 108.499999) (end 142.3 108) (width 0.3) (layer B.Cu) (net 5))
 (via (at 142.3 108) (size 0.6) (drill 0.4) (layers F.Cu B.Cu) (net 5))
 (segment (start 140.16 114.43) (end 142.47 114.43) (width 0.3) (layer F.Cu) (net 5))
 (segment (start 142.47 114.43) (end 142.5 114.4) (width 0.3) (layer F.Cu) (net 5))
 (via (at 142.5 114.4) (size 0.6) (drill 0.4) (layers F.Cu B.Cu) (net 5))
 (segment (start 142.07 108.03) (end 145.0964 105.0036) (width 0.3) (layer F.Cu) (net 5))
 (segment (start 145.0964 105.0036) (end 148.5011 105.0036) (width 0.3) (layer F.Cu) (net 5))
 (segment (start 140.16 108.03) (end 142.07 108.03) (width 0.3) (layer F.Cu) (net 5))
 (segment (start 140.16 109.13) (end 141.74999 109.13) (width 0.3) (layer F.Cu) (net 6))
 (segment (start 141.74999 109.13) (end 141.9 108.97999) (width 0.3) (layer F.Cu) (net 6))
 (segment (start 140.16 113.93) (end 141.37 113.93) (width 0.3) (layer F.Cu) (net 6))
 (segment (start 141.37 113.93) (end 141.6 113.7) (width 0.3) (layer F.Cu) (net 6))
 (segment (start 141.9 108.97999) (end 140.30999 108.97999) (width 0.3) (layer F.Cu) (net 6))
 (segment (start 140.30999 108.97999) (end 140.16 108.83) (width 0.3) (layer F.Cu) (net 6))
 (segment (start 141.6 113.7) (end 141.9 113.4) (width 0.3) (layer B.Cu) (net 6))
 (segment (start 141.9 113.4) (end 141.9 108.97999) (width 0.3) (layer B.Cu) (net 6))
 (via (at 141.9 108.97999) (size 0.6) (drill 0.4) (layers F.Cu B.Cu) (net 6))
 (segment (start 140.16 113.63) (end 141.53 113.63) (width 0.3) (layer F.Cu) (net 6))
 (segment (start 141.53 113.63) (end 141.6 113.7) (width 0.3) (layer F.Cu) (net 6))
 (via (at 141.6 113.7) (size 0.6) (drill 0.4) (layers F.Cu B.Cu) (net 6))
 (segment (start 140.16 109.13) (end 140.16 108.83) (width 0.3) (layer F.Cu) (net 6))
 (segment (start 140.16 113.63) (end 140.16 113.93) (width 0.3) (layer F.Cu) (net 6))
 (segment (start 142.77 108.83) (end 144.0564 107.5436) (width 0.3) (layer F.Cu) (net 6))
 (segment (start 144.0564 107.5436) (end 148.5011 107.5436) (width 0.3) (layer F.Cu) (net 6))
 (segment (start 140.16 108.83) (end 142.77 108.83) (width 0.3) (layer F.Cu) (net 6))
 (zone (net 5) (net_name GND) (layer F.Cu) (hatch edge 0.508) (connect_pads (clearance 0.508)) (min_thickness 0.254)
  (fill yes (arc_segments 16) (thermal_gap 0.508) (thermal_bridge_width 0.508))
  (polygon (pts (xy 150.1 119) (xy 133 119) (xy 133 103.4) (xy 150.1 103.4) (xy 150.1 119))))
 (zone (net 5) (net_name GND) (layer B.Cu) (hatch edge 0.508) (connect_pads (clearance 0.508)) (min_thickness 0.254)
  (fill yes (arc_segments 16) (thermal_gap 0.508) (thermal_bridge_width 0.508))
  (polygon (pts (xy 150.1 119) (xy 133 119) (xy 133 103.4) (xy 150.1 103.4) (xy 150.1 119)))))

